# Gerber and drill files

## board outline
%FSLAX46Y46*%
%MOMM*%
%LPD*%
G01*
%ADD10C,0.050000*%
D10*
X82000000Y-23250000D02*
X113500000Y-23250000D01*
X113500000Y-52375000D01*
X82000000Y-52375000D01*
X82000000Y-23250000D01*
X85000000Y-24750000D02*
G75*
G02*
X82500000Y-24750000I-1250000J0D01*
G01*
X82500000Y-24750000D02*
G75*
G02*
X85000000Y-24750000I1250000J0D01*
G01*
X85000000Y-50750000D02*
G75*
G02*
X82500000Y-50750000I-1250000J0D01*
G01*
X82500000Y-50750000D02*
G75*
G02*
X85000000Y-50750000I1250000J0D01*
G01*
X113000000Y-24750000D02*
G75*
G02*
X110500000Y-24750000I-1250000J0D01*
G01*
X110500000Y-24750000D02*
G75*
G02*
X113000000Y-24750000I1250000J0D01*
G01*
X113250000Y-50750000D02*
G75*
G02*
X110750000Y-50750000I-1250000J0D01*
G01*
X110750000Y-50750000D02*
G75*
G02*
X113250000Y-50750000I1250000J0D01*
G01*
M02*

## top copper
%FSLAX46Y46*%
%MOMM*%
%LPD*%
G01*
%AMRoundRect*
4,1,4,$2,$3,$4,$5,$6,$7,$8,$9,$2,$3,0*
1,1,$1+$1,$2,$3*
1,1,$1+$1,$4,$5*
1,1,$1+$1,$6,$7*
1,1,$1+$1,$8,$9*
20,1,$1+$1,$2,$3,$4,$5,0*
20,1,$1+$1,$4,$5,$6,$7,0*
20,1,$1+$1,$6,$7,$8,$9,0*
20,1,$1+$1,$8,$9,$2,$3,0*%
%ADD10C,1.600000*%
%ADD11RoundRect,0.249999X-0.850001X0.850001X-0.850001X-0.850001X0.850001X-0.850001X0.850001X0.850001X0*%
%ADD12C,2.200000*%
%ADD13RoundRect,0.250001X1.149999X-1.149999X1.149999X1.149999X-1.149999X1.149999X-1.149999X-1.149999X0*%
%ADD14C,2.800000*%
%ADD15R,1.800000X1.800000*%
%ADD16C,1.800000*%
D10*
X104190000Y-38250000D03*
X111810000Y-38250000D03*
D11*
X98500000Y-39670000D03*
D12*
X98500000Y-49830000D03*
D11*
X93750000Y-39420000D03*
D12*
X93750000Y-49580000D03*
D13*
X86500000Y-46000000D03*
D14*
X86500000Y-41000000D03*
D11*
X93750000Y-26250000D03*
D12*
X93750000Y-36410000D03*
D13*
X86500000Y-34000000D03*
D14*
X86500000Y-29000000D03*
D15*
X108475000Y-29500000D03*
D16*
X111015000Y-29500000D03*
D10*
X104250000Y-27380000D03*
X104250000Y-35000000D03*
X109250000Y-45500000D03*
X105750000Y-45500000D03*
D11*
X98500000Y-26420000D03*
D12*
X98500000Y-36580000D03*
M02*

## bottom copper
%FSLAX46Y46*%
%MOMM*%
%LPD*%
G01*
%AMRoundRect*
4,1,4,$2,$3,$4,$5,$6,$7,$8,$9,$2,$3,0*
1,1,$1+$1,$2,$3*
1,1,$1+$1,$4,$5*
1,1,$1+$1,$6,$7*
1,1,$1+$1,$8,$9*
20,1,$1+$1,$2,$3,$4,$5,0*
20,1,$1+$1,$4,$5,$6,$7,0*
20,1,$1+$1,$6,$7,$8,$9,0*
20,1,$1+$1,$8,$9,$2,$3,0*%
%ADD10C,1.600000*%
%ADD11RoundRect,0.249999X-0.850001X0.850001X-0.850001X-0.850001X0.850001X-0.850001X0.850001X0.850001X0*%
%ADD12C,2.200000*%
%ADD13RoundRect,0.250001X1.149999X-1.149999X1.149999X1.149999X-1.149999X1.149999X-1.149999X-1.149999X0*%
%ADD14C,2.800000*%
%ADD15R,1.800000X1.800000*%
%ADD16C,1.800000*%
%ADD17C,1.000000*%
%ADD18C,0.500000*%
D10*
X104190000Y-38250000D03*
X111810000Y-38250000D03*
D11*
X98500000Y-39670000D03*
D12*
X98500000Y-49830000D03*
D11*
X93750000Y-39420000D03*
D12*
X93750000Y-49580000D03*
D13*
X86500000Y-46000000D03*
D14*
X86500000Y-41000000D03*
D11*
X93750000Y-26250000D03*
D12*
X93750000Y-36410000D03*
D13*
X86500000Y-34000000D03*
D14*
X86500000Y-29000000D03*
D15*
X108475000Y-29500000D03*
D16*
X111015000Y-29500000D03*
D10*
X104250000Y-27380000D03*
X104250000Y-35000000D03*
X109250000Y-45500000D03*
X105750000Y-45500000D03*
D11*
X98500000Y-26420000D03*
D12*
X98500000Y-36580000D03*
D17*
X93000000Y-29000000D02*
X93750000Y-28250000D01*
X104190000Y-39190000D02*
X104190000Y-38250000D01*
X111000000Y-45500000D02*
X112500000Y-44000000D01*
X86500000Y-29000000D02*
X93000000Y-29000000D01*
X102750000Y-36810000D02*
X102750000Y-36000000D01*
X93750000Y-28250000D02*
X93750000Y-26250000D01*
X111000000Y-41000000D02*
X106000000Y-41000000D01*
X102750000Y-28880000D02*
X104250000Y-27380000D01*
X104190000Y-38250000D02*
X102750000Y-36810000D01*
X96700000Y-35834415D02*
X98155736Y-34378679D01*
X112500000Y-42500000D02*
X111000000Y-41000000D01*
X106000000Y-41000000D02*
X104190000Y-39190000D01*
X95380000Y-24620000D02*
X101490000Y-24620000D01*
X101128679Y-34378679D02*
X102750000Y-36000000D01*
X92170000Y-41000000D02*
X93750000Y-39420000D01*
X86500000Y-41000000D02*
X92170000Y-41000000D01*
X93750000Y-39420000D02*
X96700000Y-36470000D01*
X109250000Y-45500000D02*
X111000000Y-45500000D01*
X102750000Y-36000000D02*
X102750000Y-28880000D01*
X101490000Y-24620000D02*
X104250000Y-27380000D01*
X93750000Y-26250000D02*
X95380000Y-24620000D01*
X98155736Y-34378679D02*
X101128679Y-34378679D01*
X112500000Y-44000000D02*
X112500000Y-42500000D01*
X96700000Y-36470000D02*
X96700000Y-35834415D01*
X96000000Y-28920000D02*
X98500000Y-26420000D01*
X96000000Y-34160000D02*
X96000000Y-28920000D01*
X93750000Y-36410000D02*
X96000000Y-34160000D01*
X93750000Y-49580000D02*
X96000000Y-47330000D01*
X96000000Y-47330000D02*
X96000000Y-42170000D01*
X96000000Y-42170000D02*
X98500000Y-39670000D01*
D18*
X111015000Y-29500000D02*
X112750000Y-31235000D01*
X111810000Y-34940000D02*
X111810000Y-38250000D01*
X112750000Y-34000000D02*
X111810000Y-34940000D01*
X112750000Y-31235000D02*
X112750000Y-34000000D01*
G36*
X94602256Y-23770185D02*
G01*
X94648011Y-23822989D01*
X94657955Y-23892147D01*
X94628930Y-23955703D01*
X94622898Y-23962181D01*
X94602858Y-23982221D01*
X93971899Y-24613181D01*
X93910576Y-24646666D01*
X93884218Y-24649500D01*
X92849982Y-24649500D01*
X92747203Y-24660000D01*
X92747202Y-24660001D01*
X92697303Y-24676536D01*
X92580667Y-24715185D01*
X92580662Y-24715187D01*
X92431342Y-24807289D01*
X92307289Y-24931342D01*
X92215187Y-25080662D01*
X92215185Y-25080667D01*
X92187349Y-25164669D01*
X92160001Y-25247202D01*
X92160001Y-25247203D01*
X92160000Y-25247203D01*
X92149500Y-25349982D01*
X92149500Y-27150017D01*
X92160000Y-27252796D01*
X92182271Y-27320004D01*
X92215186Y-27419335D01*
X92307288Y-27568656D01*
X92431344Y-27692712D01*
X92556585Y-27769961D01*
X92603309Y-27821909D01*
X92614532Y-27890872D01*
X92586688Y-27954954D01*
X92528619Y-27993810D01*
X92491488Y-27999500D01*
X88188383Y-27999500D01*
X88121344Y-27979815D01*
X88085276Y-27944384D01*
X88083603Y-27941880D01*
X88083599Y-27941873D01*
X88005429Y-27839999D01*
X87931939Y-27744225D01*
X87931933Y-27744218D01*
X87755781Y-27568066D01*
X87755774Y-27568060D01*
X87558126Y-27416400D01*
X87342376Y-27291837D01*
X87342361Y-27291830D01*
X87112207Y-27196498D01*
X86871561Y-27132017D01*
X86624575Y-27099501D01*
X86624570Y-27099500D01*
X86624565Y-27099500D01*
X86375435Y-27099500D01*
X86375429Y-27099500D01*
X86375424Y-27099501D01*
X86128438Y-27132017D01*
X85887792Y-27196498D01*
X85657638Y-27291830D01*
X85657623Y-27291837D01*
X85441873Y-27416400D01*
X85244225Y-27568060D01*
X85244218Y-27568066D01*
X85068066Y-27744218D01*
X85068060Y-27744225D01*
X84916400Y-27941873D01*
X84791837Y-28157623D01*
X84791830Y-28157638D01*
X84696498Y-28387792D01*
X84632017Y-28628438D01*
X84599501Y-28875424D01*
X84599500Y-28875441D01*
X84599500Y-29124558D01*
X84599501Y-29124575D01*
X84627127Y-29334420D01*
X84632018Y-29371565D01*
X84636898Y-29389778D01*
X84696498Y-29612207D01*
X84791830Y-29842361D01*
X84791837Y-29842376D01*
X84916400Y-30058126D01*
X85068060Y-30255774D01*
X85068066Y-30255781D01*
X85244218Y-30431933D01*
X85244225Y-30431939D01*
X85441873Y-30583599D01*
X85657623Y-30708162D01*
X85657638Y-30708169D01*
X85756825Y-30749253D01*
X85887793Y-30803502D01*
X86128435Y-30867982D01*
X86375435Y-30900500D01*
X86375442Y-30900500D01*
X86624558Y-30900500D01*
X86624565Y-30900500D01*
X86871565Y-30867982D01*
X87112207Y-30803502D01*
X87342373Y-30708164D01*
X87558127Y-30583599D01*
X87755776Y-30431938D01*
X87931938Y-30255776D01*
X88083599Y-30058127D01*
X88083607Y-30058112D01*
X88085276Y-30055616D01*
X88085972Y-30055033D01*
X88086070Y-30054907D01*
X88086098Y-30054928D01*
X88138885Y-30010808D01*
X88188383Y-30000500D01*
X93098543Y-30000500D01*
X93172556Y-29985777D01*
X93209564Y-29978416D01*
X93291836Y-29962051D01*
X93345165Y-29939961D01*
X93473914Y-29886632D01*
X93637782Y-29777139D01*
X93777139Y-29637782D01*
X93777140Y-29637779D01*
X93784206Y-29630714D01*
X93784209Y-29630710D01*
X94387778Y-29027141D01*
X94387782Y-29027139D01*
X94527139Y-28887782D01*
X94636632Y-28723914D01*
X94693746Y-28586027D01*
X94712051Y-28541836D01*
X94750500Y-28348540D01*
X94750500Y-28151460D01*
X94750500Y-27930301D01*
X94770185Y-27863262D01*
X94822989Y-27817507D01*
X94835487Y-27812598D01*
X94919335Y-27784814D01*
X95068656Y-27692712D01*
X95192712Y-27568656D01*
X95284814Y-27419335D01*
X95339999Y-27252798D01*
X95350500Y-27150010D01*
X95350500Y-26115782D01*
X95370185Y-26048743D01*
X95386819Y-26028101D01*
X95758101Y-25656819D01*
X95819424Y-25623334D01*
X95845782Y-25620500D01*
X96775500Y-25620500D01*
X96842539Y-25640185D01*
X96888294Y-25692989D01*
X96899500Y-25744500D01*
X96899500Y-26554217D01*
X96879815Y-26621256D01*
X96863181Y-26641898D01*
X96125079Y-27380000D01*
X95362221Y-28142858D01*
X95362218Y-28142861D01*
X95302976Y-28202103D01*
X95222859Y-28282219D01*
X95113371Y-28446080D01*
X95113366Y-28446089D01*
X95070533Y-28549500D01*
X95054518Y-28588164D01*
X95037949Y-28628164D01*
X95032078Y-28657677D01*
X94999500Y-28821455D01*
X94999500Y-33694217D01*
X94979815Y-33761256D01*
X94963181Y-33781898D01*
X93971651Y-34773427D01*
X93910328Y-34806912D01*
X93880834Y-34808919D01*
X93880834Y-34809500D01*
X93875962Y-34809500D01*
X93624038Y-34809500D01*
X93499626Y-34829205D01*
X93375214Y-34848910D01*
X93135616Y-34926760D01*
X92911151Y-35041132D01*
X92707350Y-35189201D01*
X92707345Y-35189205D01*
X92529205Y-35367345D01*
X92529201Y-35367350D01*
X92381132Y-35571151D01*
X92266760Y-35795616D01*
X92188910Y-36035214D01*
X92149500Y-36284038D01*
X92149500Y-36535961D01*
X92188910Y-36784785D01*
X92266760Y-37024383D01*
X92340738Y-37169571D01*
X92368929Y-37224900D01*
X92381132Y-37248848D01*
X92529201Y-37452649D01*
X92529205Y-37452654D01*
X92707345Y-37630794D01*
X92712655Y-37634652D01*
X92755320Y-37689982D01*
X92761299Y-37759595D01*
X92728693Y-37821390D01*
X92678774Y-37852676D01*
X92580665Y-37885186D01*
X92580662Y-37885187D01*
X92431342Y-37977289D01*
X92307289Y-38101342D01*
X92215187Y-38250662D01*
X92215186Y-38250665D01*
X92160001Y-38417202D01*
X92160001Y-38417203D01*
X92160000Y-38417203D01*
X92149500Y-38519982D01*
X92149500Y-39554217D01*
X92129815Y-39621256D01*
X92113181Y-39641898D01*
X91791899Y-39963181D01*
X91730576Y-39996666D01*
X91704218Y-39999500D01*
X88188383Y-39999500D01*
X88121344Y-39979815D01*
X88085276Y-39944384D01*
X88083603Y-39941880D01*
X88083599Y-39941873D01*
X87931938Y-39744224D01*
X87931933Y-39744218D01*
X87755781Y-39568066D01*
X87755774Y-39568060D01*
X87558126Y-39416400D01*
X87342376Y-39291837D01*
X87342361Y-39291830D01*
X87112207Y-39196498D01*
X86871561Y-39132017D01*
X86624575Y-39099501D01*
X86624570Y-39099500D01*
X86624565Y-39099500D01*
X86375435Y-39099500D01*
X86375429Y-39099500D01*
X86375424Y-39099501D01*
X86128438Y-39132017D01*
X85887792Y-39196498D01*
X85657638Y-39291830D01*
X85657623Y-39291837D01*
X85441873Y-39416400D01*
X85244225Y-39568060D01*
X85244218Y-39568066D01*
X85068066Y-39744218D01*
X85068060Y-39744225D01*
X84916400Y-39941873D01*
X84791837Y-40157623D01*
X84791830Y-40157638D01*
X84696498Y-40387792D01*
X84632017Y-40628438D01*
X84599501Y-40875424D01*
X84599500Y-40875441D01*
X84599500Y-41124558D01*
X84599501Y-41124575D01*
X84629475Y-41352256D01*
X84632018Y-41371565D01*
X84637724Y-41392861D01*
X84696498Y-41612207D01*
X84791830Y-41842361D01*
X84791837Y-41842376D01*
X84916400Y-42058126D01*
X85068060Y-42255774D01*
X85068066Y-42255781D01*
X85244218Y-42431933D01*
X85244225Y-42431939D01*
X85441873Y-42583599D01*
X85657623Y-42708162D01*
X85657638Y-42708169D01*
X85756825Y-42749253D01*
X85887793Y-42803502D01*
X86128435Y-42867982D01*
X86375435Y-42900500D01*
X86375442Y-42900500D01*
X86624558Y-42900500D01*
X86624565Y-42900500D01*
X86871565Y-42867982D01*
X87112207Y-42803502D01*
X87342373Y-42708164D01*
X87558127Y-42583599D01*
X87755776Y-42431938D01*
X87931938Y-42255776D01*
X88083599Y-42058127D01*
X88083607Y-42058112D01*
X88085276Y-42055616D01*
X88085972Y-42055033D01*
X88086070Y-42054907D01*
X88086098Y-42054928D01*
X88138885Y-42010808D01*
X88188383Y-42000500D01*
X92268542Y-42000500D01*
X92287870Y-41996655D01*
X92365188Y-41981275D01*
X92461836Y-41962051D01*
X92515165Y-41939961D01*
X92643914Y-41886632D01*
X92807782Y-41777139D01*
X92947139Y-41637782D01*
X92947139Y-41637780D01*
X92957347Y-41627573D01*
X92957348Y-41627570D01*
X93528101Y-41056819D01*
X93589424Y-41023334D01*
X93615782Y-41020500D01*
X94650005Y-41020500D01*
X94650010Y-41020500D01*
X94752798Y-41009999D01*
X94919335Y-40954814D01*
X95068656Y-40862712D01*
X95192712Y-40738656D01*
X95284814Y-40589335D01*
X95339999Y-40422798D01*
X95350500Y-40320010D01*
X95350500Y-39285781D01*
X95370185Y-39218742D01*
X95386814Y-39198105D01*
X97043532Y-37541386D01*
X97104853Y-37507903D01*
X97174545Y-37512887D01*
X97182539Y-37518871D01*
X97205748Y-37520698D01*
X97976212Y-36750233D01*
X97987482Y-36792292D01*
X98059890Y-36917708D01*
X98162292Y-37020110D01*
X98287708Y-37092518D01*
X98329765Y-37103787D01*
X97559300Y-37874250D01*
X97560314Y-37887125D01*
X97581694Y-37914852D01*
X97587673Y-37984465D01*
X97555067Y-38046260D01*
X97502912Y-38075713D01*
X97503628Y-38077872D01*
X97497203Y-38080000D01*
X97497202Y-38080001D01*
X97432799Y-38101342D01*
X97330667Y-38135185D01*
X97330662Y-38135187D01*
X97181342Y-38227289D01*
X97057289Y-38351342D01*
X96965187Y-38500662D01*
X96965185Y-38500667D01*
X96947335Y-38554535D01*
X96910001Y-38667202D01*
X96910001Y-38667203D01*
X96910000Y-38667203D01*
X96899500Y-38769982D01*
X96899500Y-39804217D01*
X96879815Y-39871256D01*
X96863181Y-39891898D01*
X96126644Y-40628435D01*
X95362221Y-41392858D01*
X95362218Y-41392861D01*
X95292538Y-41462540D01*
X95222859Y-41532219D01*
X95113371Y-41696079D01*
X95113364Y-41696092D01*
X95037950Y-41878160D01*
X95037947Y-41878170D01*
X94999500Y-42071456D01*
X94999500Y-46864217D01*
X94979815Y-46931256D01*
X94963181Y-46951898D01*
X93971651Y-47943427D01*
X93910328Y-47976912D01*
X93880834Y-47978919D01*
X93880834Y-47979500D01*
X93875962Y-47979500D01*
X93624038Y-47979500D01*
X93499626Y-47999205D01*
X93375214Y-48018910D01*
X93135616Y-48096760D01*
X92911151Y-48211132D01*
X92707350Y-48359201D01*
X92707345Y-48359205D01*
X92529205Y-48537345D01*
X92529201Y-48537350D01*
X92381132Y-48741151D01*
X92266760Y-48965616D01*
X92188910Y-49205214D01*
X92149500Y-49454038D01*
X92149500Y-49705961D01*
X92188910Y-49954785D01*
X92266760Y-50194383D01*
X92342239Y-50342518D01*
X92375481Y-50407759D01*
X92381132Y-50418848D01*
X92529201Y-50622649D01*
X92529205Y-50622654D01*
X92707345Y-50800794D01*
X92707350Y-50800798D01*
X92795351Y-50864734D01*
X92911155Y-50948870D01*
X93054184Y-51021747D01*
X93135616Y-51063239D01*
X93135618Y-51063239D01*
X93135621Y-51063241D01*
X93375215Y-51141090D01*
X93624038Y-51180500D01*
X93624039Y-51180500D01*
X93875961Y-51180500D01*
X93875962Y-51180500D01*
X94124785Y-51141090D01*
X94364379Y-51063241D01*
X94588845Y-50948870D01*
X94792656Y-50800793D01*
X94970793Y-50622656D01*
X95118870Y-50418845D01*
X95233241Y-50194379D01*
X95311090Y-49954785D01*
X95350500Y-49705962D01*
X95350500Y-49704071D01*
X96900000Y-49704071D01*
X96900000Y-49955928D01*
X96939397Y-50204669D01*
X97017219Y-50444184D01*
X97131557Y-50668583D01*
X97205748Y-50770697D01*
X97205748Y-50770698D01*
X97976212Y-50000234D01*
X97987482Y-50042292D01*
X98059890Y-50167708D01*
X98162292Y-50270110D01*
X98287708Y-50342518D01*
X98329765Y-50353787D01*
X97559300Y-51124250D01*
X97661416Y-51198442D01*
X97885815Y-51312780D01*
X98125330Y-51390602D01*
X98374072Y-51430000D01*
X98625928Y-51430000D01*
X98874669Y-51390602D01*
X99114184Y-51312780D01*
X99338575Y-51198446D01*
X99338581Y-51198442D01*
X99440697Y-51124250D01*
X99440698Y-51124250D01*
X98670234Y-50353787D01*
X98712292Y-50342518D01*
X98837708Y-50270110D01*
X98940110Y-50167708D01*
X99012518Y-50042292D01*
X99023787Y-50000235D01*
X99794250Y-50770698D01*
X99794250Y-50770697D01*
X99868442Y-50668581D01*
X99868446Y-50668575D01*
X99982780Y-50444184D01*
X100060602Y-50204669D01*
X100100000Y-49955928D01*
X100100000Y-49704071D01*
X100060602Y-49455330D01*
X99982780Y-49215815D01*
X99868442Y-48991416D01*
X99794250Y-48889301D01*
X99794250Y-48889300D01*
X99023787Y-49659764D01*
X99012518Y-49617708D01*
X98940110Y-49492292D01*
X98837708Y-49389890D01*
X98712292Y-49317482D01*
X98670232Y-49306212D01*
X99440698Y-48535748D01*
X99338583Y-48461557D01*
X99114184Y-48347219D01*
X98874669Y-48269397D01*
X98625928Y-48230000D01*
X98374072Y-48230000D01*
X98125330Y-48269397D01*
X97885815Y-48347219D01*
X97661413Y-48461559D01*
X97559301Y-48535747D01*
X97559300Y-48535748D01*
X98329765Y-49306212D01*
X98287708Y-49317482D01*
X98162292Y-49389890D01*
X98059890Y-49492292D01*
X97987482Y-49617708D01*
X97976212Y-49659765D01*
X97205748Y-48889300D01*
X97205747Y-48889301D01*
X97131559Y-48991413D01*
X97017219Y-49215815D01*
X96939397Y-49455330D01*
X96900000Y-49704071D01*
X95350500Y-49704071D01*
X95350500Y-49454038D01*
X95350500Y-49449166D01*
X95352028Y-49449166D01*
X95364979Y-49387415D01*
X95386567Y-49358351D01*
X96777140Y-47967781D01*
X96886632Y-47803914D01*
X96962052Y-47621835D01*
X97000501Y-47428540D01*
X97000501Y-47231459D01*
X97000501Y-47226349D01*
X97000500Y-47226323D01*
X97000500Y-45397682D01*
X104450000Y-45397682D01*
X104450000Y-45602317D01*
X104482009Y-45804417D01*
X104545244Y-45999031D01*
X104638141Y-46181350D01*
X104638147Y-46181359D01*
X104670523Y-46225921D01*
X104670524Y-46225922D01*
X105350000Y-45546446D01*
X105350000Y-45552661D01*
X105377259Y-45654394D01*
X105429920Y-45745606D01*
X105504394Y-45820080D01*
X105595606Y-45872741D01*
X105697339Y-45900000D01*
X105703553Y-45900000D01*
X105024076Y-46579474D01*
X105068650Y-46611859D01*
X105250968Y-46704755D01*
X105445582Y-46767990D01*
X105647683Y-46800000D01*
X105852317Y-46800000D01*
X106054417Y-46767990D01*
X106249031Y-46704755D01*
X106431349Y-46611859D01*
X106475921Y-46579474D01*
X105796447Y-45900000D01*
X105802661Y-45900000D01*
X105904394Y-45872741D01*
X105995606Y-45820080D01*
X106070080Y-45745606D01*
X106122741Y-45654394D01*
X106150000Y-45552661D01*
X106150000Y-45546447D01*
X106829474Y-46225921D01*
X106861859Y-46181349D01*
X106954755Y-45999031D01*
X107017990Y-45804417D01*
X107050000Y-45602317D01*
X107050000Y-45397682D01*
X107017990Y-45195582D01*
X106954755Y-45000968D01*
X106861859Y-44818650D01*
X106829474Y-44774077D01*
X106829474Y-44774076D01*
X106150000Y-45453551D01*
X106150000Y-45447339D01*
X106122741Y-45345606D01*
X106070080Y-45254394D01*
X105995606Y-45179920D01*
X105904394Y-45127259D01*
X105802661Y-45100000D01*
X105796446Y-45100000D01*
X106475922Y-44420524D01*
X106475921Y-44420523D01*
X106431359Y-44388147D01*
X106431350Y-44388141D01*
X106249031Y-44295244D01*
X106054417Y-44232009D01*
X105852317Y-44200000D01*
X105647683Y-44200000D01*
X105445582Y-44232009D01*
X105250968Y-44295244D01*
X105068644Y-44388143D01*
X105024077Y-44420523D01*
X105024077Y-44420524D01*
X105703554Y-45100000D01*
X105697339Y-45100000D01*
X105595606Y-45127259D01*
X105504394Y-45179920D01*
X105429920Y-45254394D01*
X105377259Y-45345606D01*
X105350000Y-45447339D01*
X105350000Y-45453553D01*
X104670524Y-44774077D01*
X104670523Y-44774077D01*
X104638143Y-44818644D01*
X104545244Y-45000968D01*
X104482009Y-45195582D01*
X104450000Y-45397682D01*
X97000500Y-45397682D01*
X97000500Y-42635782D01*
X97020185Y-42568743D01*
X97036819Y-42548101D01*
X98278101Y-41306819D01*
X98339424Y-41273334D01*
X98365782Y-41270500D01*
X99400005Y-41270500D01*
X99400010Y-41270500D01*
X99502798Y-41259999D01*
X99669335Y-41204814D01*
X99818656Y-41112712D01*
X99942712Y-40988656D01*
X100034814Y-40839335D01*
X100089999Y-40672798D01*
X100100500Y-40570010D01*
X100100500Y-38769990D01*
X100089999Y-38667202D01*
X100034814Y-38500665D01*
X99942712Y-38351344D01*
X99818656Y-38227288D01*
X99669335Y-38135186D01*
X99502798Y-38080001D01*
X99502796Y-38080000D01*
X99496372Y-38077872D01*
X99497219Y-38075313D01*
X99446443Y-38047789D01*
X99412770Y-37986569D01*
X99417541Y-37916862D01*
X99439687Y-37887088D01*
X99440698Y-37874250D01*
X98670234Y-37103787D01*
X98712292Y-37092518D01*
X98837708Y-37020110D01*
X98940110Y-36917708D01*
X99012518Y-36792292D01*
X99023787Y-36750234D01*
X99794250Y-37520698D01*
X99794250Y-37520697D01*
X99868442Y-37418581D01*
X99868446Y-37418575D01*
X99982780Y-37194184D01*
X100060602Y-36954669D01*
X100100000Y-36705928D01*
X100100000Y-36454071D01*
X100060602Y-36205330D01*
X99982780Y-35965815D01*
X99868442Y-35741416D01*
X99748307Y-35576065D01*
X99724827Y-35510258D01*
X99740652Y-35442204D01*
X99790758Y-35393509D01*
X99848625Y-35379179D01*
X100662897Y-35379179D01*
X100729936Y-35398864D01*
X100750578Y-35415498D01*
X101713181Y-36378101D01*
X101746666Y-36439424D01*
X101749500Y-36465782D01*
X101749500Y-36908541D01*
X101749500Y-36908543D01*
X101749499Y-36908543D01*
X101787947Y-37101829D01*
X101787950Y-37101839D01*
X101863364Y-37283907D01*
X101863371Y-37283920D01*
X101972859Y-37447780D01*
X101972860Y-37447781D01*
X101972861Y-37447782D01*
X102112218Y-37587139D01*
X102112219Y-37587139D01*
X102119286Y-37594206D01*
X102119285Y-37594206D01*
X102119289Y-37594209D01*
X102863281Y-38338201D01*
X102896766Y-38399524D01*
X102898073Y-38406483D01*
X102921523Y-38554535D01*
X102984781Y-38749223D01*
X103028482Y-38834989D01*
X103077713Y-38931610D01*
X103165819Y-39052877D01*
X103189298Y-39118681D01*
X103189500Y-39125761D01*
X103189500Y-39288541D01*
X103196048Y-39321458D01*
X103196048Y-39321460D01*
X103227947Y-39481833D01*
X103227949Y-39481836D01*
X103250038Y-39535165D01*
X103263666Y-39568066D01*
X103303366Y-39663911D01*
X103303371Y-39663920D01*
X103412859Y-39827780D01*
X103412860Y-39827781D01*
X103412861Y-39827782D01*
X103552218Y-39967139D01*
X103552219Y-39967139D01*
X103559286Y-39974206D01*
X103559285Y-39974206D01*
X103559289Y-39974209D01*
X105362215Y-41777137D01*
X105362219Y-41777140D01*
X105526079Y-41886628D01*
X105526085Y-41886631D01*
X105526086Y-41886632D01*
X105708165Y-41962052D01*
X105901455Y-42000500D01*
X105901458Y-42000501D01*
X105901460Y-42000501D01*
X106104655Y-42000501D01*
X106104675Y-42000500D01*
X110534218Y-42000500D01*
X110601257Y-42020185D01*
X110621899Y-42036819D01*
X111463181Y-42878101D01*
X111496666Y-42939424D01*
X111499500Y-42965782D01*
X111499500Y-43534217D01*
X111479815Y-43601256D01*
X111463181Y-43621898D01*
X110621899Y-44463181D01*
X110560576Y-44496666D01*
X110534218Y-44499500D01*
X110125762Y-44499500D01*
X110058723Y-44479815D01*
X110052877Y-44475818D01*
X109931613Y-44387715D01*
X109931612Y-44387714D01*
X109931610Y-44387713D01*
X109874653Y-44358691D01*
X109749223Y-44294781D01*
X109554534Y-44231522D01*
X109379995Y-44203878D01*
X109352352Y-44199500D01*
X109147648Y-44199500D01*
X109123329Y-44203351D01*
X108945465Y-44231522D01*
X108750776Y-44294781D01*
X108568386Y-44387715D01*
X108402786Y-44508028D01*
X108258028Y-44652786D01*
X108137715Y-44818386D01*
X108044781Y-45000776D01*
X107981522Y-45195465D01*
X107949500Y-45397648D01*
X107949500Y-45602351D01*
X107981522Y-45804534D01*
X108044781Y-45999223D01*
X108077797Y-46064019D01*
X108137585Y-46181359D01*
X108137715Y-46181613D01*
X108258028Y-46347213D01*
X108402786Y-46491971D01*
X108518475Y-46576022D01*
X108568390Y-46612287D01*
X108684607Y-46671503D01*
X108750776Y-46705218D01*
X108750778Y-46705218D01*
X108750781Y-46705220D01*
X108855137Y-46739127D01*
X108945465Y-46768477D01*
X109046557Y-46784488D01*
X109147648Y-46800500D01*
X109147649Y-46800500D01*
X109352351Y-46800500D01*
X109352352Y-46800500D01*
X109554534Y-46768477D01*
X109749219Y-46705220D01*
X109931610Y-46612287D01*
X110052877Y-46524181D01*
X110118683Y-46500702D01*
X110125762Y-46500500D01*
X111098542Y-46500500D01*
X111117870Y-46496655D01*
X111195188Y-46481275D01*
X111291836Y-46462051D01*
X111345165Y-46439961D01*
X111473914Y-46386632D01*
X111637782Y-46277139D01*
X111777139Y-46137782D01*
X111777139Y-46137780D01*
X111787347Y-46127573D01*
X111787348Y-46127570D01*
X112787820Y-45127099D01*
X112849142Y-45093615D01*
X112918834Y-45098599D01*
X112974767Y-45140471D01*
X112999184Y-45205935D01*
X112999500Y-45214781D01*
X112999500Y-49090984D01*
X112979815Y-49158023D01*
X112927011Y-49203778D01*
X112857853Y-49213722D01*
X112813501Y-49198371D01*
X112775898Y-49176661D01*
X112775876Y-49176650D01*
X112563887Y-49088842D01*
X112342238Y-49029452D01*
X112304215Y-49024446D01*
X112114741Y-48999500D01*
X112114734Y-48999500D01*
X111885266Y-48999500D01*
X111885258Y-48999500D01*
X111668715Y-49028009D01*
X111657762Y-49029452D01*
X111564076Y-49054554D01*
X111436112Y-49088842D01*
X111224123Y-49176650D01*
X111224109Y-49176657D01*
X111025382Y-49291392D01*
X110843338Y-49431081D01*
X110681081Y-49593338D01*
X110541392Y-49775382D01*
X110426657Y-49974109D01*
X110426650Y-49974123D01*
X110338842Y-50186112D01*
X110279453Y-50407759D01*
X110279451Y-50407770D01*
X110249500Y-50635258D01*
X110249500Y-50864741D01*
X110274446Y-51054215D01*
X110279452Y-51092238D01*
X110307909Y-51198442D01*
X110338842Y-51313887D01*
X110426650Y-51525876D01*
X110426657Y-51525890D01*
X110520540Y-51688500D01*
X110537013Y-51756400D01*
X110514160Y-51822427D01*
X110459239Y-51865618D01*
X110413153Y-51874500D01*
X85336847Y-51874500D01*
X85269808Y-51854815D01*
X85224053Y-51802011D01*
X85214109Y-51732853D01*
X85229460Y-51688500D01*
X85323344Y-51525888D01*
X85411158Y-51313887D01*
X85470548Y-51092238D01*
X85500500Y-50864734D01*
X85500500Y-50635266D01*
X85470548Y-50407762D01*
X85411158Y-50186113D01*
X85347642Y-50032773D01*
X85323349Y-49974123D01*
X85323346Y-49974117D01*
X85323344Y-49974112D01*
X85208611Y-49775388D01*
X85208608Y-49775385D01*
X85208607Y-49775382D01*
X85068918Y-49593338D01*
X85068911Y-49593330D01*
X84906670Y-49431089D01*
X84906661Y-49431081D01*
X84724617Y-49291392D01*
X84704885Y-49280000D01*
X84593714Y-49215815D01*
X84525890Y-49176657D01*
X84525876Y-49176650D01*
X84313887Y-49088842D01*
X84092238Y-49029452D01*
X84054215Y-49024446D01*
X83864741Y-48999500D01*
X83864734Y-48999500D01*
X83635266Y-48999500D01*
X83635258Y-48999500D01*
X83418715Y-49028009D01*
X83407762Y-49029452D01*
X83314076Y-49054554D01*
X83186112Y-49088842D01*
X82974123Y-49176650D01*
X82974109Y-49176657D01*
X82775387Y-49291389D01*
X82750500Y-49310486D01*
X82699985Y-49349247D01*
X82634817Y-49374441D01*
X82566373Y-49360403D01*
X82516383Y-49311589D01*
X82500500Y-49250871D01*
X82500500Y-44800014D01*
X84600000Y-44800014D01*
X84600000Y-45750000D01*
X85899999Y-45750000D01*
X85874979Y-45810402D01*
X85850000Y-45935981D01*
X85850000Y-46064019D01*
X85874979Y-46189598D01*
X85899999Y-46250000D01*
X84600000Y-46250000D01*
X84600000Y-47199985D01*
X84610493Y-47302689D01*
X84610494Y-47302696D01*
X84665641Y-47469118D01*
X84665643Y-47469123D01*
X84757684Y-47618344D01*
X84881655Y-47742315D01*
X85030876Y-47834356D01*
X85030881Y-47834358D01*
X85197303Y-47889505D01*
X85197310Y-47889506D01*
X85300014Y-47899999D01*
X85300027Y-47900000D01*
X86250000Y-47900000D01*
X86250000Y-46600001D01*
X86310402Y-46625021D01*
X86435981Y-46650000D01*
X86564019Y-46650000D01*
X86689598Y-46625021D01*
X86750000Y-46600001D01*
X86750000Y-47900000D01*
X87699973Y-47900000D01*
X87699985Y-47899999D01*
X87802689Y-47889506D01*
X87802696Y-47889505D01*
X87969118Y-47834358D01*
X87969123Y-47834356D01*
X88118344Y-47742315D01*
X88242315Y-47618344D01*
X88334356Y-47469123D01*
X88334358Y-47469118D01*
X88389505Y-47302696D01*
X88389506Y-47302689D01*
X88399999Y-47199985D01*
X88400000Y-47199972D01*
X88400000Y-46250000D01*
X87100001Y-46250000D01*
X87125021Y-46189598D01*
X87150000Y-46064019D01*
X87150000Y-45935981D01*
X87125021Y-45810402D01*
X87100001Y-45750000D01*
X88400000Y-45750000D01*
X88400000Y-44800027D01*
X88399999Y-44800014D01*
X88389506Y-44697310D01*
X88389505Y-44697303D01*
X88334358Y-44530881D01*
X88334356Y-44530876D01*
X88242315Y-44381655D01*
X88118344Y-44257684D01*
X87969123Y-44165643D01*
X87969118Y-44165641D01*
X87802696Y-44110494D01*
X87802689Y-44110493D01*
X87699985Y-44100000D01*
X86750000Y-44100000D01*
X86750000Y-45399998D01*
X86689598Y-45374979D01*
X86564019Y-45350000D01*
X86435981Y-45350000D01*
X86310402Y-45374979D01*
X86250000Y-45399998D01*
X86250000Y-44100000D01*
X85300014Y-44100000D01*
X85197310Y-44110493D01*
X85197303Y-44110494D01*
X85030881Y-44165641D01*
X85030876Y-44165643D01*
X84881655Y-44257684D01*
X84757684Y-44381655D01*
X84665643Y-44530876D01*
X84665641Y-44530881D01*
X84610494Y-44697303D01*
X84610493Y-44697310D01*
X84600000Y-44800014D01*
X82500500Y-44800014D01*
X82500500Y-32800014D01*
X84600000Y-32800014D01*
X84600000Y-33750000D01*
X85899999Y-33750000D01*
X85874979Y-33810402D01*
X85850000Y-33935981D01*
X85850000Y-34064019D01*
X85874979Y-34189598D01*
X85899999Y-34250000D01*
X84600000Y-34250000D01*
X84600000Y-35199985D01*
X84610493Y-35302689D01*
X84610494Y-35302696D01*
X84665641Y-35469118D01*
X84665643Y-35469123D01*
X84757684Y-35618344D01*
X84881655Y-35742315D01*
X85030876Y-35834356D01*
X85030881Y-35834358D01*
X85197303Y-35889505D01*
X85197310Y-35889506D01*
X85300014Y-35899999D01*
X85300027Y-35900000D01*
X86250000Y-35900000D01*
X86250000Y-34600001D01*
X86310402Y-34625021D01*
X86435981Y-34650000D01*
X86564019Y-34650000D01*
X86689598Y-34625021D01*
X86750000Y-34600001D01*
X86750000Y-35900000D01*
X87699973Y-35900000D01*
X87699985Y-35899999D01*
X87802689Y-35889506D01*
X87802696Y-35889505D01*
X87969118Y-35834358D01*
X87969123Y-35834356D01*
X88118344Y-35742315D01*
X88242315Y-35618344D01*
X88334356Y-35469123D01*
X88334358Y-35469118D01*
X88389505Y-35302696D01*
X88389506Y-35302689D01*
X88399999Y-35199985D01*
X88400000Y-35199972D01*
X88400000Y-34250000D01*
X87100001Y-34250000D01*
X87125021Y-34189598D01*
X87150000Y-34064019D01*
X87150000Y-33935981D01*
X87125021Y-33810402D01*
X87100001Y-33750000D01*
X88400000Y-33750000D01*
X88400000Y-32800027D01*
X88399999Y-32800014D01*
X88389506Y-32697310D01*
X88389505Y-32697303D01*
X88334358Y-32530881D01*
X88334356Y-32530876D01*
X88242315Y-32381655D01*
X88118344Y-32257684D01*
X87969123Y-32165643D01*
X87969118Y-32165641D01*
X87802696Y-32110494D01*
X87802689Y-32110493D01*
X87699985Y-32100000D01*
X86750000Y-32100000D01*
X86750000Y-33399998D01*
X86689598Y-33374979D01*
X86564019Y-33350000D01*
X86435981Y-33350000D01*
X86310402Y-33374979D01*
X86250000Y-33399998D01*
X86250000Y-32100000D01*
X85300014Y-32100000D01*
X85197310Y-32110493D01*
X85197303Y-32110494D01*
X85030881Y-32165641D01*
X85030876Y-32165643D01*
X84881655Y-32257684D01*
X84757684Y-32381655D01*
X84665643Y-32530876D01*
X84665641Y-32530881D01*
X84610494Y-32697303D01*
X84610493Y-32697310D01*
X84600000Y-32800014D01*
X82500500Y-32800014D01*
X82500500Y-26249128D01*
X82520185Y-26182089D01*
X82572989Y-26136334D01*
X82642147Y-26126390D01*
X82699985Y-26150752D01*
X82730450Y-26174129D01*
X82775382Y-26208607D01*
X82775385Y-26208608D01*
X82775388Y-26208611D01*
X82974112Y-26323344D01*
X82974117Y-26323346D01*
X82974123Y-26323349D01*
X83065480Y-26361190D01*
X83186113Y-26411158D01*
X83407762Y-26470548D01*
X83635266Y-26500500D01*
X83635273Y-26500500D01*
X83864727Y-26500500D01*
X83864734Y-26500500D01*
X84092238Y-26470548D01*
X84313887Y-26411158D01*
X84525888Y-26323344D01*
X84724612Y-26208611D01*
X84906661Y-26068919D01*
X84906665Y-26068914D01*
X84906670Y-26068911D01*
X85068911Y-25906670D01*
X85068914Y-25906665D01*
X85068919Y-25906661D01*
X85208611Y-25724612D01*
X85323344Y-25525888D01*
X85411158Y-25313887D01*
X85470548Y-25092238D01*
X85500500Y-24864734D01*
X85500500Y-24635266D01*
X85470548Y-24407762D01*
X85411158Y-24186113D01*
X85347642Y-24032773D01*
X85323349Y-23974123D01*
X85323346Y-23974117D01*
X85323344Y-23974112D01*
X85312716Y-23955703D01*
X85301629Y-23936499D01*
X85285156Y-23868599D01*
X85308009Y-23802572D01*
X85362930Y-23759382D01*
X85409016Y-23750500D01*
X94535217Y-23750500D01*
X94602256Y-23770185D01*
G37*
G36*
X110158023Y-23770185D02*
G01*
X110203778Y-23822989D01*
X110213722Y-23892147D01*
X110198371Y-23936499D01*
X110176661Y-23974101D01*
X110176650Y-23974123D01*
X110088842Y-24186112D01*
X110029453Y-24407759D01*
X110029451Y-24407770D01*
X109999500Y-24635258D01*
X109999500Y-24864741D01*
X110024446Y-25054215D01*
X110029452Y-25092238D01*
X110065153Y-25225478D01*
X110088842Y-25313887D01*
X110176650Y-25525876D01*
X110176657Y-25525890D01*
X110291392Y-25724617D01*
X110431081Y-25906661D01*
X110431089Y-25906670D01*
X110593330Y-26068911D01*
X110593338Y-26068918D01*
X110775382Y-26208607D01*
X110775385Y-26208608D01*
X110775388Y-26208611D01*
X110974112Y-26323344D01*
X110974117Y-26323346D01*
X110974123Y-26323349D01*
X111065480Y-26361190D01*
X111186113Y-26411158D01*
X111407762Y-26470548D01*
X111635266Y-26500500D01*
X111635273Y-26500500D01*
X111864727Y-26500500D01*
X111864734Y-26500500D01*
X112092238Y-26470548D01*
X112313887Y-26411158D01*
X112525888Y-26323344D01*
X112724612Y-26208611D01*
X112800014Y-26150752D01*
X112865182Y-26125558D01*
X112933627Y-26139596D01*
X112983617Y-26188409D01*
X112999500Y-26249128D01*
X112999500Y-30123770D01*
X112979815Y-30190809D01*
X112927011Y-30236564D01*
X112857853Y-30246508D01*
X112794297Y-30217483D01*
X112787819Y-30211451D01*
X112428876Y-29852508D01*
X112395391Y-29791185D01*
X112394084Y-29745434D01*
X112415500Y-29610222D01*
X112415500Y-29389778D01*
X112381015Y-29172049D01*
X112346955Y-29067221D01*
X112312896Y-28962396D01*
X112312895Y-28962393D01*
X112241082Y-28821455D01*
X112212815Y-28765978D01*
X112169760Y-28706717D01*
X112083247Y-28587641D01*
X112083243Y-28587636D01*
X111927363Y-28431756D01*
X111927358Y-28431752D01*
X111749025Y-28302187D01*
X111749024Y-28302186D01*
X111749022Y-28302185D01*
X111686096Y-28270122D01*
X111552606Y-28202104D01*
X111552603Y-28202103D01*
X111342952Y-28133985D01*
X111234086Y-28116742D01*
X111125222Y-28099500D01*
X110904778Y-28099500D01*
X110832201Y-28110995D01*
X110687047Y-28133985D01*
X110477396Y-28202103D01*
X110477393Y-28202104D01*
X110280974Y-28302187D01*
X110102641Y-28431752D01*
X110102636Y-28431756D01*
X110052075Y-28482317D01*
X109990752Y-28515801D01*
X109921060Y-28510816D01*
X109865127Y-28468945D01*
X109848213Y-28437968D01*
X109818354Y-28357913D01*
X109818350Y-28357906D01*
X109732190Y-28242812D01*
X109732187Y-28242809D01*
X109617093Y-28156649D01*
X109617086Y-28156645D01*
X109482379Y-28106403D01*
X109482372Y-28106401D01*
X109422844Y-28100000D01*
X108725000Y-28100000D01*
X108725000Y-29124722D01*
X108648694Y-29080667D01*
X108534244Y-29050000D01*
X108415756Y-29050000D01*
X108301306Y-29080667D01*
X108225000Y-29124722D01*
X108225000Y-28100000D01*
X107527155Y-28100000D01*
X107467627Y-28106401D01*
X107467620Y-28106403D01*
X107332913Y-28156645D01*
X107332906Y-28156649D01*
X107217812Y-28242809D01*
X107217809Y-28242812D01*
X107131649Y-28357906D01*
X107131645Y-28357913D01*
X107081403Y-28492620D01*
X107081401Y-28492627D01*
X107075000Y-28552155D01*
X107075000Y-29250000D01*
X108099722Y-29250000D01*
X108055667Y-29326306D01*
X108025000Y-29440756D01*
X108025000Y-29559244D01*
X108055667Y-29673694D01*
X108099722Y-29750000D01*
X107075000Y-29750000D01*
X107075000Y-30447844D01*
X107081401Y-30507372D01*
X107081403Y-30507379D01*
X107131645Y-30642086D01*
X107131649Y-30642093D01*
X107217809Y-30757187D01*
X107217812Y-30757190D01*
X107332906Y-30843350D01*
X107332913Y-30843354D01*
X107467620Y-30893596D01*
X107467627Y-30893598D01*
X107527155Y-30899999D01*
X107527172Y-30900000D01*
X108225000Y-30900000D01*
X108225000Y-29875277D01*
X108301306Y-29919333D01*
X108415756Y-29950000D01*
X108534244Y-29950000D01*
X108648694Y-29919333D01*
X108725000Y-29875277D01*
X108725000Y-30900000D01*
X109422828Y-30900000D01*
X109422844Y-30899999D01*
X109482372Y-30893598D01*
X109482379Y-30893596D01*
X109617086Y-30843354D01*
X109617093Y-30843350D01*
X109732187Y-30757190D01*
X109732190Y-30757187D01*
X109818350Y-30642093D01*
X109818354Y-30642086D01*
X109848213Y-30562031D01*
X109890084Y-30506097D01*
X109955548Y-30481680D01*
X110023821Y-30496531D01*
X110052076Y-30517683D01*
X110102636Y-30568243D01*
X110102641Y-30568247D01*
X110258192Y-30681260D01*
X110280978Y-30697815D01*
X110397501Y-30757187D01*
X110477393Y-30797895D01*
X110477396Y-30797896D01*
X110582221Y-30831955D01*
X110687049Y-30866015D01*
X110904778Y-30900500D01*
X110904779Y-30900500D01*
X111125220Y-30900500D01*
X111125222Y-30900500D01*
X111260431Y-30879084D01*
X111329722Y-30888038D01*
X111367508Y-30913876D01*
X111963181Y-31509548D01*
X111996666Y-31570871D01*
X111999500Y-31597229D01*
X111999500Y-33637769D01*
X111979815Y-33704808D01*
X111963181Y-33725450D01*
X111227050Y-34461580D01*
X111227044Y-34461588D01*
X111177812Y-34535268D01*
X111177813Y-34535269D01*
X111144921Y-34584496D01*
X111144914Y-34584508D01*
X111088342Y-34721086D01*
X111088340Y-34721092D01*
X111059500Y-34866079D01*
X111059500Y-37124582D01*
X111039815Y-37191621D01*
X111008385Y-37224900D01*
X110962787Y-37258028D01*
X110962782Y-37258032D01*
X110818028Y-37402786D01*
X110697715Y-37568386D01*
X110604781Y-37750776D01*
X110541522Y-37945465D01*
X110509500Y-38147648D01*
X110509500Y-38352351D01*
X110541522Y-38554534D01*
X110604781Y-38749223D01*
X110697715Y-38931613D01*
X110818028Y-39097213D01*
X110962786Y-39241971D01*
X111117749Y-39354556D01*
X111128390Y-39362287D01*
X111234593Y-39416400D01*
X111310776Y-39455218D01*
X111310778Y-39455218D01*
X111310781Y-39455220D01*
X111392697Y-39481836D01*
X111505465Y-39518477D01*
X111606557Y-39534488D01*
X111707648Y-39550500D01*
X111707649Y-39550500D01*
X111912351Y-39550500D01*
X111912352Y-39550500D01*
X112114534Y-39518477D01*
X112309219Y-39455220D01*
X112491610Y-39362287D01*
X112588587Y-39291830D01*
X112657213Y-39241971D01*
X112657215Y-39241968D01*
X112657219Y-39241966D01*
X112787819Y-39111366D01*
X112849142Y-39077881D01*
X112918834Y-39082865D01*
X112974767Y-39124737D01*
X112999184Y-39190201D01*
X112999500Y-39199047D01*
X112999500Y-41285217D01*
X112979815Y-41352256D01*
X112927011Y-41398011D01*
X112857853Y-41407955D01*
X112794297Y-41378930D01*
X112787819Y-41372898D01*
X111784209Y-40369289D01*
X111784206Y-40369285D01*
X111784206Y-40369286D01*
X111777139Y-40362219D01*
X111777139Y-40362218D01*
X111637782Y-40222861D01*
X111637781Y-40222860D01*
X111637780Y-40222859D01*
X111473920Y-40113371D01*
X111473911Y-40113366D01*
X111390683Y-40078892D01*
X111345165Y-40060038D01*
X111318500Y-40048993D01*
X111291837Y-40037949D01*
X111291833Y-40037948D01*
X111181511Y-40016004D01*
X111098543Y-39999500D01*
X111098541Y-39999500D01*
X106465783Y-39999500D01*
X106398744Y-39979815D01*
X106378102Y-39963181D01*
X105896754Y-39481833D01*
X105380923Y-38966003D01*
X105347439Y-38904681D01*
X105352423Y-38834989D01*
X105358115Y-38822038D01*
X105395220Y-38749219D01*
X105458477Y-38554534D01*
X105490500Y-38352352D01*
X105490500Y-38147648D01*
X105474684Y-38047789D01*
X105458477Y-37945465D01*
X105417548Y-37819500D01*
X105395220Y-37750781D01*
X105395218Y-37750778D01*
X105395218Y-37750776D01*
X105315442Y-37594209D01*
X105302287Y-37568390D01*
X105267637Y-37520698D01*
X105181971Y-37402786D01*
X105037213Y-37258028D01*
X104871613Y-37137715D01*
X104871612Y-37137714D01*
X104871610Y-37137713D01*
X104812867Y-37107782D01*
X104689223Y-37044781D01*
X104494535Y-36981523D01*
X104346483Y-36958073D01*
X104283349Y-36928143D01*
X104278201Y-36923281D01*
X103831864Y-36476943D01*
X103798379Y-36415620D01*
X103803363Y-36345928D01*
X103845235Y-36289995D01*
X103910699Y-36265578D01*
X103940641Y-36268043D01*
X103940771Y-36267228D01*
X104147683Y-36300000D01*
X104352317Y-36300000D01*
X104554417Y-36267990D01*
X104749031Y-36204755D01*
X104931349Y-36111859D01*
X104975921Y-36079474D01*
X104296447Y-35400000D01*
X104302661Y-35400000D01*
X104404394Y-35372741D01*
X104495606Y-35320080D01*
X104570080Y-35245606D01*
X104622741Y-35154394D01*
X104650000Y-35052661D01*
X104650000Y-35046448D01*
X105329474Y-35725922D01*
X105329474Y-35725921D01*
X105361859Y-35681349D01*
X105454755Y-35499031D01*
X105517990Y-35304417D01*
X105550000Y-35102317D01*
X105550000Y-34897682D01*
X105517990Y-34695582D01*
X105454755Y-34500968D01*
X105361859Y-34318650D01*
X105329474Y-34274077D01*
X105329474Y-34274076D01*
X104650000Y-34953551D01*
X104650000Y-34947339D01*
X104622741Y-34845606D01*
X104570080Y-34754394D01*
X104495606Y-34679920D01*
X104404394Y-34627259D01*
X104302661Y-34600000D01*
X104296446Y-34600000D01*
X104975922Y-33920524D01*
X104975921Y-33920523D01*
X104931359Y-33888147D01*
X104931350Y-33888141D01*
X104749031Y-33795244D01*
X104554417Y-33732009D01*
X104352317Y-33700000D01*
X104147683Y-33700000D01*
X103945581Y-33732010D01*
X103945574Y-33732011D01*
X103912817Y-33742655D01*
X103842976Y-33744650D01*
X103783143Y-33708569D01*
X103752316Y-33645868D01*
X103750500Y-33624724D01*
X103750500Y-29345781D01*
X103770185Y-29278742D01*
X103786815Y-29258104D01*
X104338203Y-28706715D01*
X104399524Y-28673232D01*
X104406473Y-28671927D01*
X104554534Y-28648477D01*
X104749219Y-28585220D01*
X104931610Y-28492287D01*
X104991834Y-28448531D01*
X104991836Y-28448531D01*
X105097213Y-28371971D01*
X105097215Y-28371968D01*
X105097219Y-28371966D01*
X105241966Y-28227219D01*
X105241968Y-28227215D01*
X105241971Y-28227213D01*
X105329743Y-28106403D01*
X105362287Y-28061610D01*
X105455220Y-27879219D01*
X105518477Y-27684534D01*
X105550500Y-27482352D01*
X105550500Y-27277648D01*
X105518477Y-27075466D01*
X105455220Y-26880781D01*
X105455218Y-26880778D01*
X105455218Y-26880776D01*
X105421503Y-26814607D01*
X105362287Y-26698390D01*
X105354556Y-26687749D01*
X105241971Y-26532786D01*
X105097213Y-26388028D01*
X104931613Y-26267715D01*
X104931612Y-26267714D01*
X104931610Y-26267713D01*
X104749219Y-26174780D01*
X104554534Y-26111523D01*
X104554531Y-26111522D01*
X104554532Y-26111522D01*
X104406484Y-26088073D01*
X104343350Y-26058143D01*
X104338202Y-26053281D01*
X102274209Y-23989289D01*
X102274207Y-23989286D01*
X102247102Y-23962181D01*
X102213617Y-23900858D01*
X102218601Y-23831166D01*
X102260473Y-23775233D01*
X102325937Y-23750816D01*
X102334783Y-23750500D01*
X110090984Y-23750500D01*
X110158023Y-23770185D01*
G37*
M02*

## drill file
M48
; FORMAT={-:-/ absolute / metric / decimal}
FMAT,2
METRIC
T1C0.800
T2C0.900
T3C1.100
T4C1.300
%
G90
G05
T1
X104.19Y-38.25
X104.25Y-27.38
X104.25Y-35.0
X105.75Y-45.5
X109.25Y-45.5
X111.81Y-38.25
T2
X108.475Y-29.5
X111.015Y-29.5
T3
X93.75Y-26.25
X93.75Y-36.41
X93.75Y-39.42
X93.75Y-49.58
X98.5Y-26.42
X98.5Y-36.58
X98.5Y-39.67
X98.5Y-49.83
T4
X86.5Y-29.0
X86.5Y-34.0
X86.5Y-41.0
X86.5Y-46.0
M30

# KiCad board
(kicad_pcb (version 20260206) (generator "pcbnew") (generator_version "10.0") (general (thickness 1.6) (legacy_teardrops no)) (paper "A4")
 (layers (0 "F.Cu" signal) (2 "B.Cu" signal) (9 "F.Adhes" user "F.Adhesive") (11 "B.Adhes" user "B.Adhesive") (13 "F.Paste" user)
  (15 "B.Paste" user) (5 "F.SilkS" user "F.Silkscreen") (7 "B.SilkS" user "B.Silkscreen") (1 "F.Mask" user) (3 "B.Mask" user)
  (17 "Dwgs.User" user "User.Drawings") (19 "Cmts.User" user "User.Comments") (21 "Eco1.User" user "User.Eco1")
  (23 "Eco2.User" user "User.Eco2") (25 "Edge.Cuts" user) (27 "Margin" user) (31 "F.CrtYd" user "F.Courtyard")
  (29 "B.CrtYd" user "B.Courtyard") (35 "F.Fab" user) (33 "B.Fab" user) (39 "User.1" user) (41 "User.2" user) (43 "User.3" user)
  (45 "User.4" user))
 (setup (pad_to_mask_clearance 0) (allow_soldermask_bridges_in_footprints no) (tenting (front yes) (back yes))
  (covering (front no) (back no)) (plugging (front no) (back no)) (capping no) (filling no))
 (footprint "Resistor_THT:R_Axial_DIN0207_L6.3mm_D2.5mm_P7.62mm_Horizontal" (layer "F.Cu") (at 104.19 38.25)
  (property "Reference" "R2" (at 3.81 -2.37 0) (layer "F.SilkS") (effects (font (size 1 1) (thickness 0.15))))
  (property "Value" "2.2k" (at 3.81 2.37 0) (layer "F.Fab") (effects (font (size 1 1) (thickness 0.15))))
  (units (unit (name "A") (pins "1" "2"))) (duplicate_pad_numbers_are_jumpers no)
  (pad "1" thru_hole circle (at 0 0) (size 1.6 1.6) (drill 0.8) (layers "*.Cu" "*.Mask") (remove_unused_layers no) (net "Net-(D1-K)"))
  (pad "2" thru_hole circle (at 7.62 0) (size 1.6 1.6) (drill 0.8) (layers "*.Cu" "*.Mask") (remove_unused_layers no) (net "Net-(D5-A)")))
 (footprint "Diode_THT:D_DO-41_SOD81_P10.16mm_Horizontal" (layer "F.Cu") (at 98.5 39.67 -90)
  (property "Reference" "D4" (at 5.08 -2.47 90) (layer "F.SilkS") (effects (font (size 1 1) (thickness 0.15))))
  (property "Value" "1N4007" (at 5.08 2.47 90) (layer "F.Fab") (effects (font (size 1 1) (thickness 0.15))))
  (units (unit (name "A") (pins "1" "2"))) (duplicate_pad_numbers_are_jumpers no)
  (pad "1" thru_hole roundrect (at 0 0 270) (size 2.2 2.2) (drill 1.1) (layers "*.Cu" "*.Mask") (remove_unused_layers no)
   (roundrect_rratio 0.113636) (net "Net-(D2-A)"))
  (pad "2" thru_hole circle (at 10.16 0 270) (size 2.2 2.2) (drill 1.1) (layers "*.Cu" "*.Mask") (remove_unused_layers no) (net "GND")))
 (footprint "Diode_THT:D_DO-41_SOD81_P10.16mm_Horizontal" (layer "F.Cu") (at 93.75 39.42 -90)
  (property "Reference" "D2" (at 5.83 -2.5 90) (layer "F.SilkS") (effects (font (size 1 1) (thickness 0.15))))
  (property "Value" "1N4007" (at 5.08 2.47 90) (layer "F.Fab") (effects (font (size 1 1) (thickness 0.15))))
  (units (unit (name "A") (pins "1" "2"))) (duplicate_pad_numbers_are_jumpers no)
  (pad "1" thru_hole roundrect (at 0 0 270) (size 2.2 2.2) (drill 1.1) (layers "*.Cu" "*.Mask") (remove_unused_layers no)
   (roundrect_rratio 0.113636) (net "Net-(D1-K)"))
  (pad "2" thru_hole circle (at 10.16 0 270) (size 2.2 2.2) (drill 1.1) (layers "*.Cu" "*.Mask") (remove_unused_layers no)
   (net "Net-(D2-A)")))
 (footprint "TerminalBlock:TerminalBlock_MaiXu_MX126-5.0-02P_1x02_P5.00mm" (layer "F.Cu") (at 86.5 46 90)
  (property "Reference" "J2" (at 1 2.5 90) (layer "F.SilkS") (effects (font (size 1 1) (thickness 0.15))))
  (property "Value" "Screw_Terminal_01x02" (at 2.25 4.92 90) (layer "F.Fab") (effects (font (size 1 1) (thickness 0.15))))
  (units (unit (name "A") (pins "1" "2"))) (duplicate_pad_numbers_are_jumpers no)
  (pad "1" thru_hole roundrect (at 0 0 90) (size 2.8 2.8) (drill 1.3) (layers "*.Cu" "*.Mask") (remove_unused_layers no)
   (roundrect_rratio 0.089286) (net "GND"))
  (pad "2" thru_hole circle (at 5 0 90) (size 2.8 2.8) (drill 1.3) (layers "*.Cu" "*.Mask") (remove_unused_layers no) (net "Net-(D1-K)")))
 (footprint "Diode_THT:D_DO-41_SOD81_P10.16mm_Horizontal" (layer "F.Cu") (at 93.75 26.25 -90)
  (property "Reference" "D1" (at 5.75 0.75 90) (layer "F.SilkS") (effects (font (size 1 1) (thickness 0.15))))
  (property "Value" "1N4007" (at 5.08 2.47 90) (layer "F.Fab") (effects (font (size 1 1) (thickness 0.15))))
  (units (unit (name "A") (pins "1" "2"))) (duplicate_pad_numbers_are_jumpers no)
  (pad "1" thru_hole roundrect (at 0 0 270) (size 2.2 2.2) (drill 1.1) (layers "*.Cu" "*.Mask") (remove_unused_layers no)
   (roundrect_rratio 0.113636) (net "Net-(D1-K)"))
  (pad "2" thru_hole circle (at 10.16 0 270) (size 2.2 2.2) (drill 1.1) (layers "*.Cu" "*.Mask") (remove_unused_layers no)
   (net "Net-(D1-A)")))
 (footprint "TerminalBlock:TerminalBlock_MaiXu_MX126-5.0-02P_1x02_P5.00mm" (layer "F.Cu") (at 86.5 34 90)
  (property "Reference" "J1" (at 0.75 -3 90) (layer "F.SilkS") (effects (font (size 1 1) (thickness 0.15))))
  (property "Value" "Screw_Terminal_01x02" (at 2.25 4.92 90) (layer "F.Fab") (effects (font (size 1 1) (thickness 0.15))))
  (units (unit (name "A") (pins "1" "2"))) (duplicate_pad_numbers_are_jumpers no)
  (pad "1" thru_hole roundrect (at 0 0 90) (size 2.8 2.8) (drill 1.3) (layers "*.Cu" "*.Mask") (remove_unused_layers no)
   (roundrect_rratio 0.089286) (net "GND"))
  (pad "2" thru_hole circle (at 5 0 90) (size 2.8 2.8) (drill 1.3) (layers "*.Cu" "*.Mask") (remove_unused_layers no) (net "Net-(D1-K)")))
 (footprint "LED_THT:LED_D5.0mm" (layer "F.Cu") (at 108.475 29.5)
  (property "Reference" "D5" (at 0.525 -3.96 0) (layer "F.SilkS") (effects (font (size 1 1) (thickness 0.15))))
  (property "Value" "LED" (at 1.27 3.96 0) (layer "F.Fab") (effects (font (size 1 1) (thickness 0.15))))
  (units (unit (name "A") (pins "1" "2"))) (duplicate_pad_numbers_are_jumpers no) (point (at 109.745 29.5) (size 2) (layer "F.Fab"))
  (pad "1" thru_hole rect (at 0 0) (size 1.8 1.8) (drill 0.9) (layers "*.Cu" "*.Mask") (remove_unused_layers no) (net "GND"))
  (pad "2" thru_hole circle (at 2.54 0) (size 1.8 1.8) (drill 0.9) (layers "*.Cu" "*.Mask") (remove_unused_layers no) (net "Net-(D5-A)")))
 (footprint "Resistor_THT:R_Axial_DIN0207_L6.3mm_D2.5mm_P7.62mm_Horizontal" (layer "F.Cu") (at 104.25 27.38 -90)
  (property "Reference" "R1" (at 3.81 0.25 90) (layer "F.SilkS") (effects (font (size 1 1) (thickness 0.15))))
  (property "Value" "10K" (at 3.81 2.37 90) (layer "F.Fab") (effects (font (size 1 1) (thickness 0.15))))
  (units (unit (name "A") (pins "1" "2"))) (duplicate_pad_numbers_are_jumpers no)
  (pad "1" thru_hole circle (at 0 0 270) (size 1.6 1.6) (drill 0.8) (layers "*.Cu" "*.Mask") (remove_unused_layers no) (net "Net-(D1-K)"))
  (pad "2" thru_hole circle (at 7.62 0 270) (size 1.6 1.6) (drill 0.8) (layers "*.Cu" "*.Mask") (remove_unused_layers no) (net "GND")))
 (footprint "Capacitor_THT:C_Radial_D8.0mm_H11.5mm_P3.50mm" (layer "F.Cu") (at 109.25 45.5 180)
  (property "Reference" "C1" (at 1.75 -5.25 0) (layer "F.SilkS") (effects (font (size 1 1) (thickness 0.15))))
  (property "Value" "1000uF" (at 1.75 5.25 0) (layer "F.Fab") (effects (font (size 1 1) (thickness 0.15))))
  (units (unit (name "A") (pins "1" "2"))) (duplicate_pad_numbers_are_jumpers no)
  (pad "1" thru_hole circle (at 0 0 180) (size 1.6 1.6) (drill 0.8) (layers "*.Cu" "*.Mask") (remove_unused_layers no) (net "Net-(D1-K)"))
  (pad "2" thru_hole circle (at 3.5 0 180) (size 1.6 1.6) (drill 0.8) (layers "*.Cu" "*.Mask") (remove_unused_layers no) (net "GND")))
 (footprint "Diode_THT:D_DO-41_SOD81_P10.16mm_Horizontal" (layer "F.Cu") (at 98.5 26.42 -90)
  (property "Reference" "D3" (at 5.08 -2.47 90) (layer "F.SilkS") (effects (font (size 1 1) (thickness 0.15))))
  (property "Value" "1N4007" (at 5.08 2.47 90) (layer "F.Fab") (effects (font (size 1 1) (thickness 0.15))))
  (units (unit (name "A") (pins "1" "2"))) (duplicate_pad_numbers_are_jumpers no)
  (pad "1" thru_hole roundrect (at 0 0 270) (size 2.2 2.2) (drill 1.1) (layers "*.Cu" "*.Mask") (remove_unused_layers no)
   (roundrect_rratio 0.113636) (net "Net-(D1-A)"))
  (pad "2" thru_hole circle (at 10.16 0 270) (size 2.2 2.2) (drill 1.1) (layers "*.Cu" "*.Mask") (remove_unused_layers no) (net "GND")))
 (gr_rect (start 82 23.25) (end 113.5 52.375) (stroke (width 0.05) (type default)) (fill no) (layer "Edge.Cuts"))
 (gr_circle (center 83.75 24.75) (end 84.75 25.5) (stroke (width 0.05) (type default)) (fill no) (layer "Edge.Cuts"))
 (gr_circle (center 83.75 50.75) (end 84.75 51.5) (stroke (width 0.05) (type default)) (fill no) (layer "Edge.Cuts"))
 (gr_circle (center 111.75 24.75) (end 112.75 25.5) (stroke (width 0.05) (type default)) (fill no) (layer "Edge.Cuts"))
 (gr_circle (center 112 50.75) (end 113 51.5) (stroke (width 0.05) (type default)) (fill no) (layer "Edge.Cuts"))
 (segment (start 93 29) (end 93.75 28.25) (width 1) (layer "B.Cu") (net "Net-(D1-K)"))
 (segment (start 104.19 39.19) (end 104.19 38.25) (width 1) (layer "B.Cu") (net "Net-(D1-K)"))
 (segment (start 111 45.5) (end 112.5 44) (width 1) (layer "B.Cu") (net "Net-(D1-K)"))
 (segment (start 86.5 29) (end 93 29) (width 1) (layer "B.Cu") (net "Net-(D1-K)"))
 (segment (start 102.75 36.81) (end 102.75 36) (width 1) (layer "B.Cu") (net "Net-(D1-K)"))
 (segment (start 93.75 28.25) (end 93.75 26.25) (width 1) (layer "B.Cu") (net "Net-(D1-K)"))
 (segment (start 111 41) (end 106 41) (width 1) (layer "B.Cu") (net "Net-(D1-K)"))
 (segment (start 102.75 28.88) (end 104.25 27.38) (width 1) (layer "B.Cu") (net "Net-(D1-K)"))
 (segment (start 104.19 38.25) (end 102.75 36.81) (width 1) (layer "B.Cu") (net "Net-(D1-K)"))
 (segment (start 96.7 35.834415) (end 98.155736 34.378679) (width 1) (layer "B.Cu") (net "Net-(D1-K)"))
 (segment (start 112.5 42.5) (end 111 41) (width 1) (layer "B.Cu") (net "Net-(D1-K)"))
 (segment (start 106 41) (end 104.19 39.19) (width 1) (layer "B.Cu") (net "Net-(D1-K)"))
 (segment (start 95.38 24.62) (end 101.49 24.62) (width 1) (layer "B.Cu") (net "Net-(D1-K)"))
 (segment (start 101.128679 34.378679) (end 102.75 36) (width 1) (layer "B.Cu") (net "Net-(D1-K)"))
 (segment (start 92.17 41) (end 93.75 39.42) (width 1) (layer "B.Cu") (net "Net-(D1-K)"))
 (segment (start 86.5 41) (end 92.17 41) (width 1) (layer "B.Cu") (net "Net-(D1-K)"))
 (segment (start 93.75 39.42) (end 96.7 36.47) (width 1) (layer "B.Cu") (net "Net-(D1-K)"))
 (segment (start 109.25 45.5) (end 111 45.5) (width 1) (layer "B.Cu") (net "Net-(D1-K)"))
 (segment (start 102.75 36) (end 102.75 28.88) (width 1) (layer "B.Cu") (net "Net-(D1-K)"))
 (segment (start 101.49 24.62) (end 104.25 27.38) (width 1) (layer "B.Cu") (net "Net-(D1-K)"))
 (segment (start 93.75 26.25) (end 95.38 24.62) (width 1) (layer "B.Cu") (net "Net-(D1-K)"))
 (segment (start 98.155736 34.378679) (end 101.128679 34.378679) (width 1) (layer "B.Cu") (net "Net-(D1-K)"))
 (segment (start 112.5 44) (end 112.5 42.5) (width 1) (layer "B.Cu") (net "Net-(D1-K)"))
 (segment (start 96.7 36.47) (end 96.7 35.834415) (width 1) (layer "B.Cu") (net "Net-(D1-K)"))
 (segment (start 96 28.92) (end 98.5 26.42) (width 1) (layer "B.Cu") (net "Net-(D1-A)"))
 (segment (start 96 34.16) (end 96 28.92) (width 1) (layer "B.Cu") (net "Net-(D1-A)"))
 (segment (start 93.75 36.41) (end 96 34.16) (width 1) (layer "B.Cu") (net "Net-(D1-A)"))
 (segment (start 93.75 49.58) (end 96 47.33) (width 1) (layer "B.Cu") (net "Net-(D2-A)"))
 (segment (start 96 47.33) (end 96 42.17) (width 1) (layer "B.Cu") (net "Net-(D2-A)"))
 (segment (start 96 42.17) (end 98.5 39.67) (width 1) (layer "B.Cu") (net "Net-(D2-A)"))
 (segment (start 111.015 29.5) (end 112.75 31.235) (width 0.5) (layer "B.Cu") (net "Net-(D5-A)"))
 (segment (start 111.81 34.94) (end 111.81 38.25) (width 0.5) (layer "B.Cu") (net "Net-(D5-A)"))
 (segment (start 112.75 34) (end 111.81 34.94) (width 0.5) (layer "B.Cu") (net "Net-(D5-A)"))
 (segment (start 112.75 31.235) (end 112.75 34) (width 0.5) (layer "B.Cu") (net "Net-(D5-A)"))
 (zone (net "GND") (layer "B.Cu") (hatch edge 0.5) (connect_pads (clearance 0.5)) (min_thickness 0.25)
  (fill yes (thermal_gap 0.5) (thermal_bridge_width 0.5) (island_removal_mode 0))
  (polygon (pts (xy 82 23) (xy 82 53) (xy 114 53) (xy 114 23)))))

